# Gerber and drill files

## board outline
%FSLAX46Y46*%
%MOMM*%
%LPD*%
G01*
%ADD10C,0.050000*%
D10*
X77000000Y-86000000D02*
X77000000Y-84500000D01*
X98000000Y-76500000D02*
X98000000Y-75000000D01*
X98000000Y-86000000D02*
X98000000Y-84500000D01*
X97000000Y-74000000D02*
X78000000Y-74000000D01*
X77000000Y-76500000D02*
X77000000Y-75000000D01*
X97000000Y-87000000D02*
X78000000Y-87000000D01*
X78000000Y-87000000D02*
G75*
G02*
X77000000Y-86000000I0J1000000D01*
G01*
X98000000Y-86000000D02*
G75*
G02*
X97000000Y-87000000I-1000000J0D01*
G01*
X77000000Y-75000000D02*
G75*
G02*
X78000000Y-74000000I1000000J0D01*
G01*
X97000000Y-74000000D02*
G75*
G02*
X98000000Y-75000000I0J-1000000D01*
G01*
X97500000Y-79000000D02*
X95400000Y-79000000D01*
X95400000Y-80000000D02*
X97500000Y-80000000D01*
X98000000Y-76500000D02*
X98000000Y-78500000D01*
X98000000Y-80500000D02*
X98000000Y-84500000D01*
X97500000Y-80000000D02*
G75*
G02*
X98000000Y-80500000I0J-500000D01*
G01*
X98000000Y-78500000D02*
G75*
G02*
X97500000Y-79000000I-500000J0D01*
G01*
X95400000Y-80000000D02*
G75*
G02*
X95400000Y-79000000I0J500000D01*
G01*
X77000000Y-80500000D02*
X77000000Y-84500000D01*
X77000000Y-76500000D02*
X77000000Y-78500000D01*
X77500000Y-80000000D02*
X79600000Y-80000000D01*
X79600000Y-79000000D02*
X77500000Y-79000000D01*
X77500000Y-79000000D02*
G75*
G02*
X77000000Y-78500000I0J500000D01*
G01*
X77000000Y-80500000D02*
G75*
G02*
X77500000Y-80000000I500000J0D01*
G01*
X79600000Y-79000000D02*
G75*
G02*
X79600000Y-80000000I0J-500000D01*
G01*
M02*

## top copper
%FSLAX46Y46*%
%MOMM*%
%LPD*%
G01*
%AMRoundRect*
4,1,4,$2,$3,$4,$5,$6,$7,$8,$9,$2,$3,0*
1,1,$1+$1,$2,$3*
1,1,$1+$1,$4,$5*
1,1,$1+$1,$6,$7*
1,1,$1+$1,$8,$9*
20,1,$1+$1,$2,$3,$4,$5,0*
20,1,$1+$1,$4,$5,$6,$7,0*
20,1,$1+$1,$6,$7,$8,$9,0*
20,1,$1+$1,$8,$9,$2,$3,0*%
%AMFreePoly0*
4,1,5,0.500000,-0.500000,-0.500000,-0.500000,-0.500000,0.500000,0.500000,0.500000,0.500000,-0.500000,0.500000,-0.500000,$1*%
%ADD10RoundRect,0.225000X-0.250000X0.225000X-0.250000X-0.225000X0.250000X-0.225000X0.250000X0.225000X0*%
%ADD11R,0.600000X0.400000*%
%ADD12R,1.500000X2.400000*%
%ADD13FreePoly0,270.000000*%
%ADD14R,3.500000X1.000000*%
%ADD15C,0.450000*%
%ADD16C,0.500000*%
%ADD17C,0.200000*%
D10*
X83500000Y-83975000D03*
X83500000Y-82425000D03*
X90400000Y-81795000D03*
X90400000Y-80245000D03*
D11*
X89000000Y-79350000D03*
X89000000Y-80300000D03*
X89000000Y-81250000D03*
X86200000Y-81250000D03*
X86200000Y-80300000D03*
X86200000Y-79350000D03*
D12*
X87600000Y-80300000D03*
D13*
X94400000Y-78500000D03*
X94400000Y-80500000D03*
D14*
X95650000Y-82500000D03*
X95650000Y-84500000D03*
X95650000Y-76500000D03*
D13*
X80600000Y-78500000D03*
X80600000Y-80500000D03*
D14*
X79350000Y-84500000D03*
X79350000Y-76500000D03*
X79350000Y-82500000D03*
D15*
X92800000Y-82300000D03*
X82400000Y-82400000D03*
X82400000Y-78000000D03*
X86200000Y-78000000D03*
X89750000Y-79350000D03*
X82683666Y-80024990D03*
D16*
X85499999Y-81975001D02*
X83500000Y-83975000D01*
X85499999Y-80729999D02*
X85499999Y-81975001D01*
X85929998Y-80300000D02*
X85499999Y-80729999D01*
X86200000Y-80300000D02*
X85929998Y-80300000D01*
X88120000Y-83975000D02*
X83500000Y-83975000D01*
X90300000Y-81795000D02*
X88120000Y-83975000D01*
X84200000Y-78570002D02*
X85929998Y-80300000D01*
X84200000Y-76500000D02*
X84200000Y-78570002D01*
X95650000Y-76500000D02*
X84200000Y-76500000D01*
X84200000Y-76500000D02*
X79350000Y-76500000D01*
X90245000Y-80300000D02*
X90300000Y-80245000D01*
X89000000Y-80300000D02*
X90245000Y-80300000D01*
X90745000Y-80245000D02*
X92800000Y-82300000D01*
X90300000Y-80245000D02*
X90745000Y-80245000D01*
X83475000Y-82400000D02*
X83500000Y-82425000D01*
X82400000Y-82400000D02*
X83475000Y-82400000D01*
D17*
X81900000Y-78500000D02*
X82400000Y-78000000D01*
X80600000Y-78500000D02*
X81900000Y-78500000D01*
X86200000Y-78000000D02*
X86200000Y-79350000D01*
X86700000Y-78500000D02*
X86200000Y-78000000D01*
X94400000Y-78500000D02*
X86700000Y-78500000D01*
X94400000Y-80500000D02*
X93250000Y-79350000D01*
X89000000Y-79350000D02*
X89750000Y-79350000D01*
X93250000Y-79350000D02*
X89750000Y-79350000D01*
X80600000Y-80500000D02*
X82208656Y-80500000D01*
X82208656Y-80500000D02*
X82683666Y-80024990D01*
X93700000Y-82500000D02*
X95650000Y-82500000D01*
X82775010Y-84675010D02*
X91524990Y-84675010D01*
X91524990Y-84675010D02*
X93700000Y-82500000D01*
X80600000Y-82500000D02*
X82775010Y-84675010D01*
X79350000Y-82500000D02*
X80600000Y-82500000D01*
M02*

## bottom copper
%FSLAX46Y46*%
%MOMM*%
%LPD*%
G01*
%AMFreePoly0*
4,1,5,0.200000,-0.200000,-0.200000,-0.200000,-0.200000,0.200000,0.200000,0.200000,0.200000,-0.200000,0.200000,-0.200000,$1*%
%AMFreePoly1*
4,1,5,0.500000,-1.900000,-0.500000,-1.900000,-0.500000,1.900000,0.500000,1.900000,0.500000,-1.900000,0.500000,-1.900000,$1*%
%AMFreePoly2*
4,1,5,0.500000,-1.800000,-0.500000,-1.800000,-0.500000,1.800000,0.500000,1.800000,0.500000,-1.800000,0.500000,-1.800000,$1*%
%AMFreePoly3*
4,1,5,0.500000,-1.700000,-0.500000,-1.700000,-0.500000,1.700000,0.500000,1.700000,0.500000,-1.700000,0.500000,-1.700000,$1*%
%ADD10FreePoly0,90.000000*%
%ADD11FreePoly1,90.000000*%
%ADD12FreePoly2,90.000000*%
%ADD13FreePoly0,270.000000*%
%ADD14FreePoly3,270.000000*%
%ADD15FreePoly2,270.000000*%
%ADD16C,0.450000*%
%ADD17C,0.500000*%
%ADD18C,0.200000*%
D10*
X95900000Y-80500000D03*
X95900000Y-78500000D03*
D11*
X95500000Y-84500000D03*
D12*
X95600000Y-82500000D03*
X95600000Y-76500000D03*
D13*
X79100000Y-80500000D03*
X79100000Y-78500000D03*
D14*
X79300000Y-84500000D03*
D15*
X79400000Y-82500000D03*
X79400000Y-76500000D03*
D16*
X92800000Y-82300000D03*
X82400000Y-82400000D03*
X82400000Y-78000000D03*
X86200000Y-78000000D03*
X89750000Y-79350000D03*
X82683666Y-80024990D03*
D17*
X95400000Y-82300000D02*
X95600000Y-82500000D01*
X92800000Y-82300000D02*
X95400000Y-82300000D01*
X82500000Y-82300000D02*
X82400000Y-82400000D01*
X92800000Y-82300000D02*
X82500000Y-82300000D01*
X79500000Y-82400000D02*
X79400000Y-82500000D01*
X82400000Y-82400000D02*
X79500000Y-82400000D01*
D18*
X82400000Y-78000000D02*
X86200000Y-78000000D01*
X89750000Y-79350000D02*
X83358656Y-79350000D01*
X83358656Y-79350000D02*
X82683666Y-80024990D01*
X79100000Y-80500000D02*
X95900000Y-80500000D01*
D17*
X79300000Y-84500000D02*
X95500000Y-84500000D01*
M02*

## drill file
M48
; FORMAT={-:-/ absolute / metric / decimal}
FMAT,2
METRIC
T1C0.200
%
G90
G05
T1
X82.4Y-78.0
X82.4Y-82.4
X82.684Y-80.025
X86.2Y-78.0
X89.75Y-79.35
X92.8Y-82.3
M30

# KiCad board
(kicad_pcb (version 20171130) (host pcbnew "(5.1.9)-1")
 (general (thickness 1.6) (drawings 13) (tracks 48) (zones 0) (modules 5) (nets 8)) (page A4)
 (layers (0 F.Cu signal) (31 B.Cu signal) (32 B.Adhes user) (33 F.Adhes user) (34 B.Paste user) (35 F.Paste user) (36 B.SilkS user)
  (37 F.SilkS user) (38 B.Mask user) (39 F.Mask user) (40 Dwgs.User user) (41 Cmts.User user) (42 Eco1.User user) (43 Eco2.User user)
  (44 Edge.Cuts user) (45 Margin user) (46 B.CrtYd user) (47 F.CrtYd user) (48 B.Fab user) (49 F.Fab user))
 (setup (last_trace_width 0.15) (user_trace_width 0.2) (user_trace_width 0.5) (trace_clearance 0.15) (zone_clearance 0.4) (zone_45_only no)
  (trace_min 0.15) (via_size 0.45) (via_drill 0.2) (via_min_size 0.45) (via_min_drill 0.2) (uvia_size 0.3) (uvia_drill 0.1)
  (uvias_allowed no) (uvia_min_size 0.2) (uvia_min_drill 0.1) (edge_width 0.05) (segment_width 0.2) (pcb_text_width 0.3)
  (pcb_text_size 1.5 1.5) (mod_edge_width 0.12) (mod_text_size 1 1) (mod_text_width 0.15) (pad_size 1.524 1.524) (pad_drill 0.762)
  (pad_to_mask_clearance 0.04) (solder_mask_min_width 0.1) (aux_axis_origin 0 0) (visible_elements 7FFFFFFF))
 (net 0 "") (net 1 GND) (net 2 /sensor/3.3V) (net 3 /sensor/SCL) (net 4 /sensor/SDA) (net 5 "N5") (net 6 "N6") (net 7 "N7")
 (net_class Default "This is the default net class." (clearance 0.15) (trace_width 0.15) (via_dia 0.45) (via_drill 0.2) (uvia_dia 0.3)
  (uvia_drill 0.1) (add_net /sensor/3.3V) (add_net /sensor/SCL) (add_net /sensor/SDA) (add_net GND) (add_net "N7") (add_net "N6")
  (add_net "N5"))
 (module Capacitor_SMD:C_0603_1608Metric (layer F.Cu) (at 83.5 83.2 270)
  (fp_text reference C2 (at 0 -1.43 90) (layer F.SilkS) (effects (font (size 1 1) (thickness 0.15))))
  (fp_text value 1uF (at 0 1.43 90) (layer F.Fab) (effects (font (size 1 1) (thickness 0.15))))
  (pad 2 smd roundrect (at 0.775 0 270) (size 0.9 0.95) (layers F.Cu F.Paste F.Mask) (roundrect_rratio 0.25) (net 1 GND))
  (pad 1 smd roundrect (at -0.775 0 270) (size 0.9 0.95) (layers F.Cu F.Paste F.Mask) (roundrect_rratio 0.25) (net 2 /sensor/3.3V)))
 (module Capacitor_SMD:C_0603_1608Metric (layer F.Cu) (at 90.4 81.02 270)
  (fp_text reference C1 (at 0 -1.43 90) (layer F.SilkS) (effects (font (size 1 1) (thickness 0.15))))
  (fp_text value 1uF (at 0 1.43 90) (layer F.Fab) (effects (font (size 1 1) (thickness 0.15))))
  (pad 2 smd roundrect (at 0.775 0 270) (size 0.9 0.95) (layers F.Cu F.Paste F.Mask) (roundrect_rratio 0.25) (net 1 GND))
  (pad 1 smd roundrect (at -0.775 0 270) (size 0.9 0.95) (layers F.Cu F.Paste F.Mask) (roundrect_rratio 0.25) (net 2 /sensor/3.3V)))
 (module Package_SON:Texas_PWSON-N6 (layer F.Cu) (at 87.6 80.3)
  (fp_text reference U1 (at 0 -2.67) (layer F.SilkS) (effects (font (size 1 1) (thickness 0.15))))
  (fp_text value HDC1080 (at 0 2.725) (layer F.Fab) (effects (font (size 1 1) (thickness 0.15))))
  (pad 6 smd rect (at 1.4 -0.95) (size 0.6 0.4) (layers F.Cu F.Paste F.Mask) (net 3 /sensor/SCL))
  (pad 5 smd rect (at 1.4 0) (size 0.6 0.4) (layers F.Cu F.Paste F.Mask) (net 2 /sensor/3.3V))
  (pad 4 smd rect (at 1.4 0.95) (size 0.6 0.4) (layers F.Cu F.Paste F.Mask))
  (pad 3 smd rect (at -1.4 0.95) (size 0.6 0.4) (layers F.Cu F.Paste F.Mask))
  (pad 2 smd rect (at -1.4 0) (size 0.6 0.4) (layers F.Cu F.Paste F.Mask) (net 1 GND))
  (pad 1 smd rect (at -1.4 -0.95) (size 0.6 0.4) (layers F.Cu F.Paste F.Mask) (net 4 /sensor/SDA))
  (pad 7 smd rect (at 0 0) (size 1.5 2.4) (layers F.Cu F.Paste F.Mask)))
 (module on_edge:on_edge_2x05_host (layer F.Cu) (at 98 80.5 270)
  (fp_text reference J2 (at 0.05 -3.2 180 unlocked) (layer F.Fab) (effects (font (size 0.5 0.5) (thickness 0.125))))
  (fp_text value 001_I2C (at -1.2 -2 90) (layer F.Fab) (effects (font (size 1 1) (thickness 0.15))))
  (fp_line (start -1.5 0.5) (end -1.5 2.6) (layer Edge.Cuts) (width 0.05))
  (fp_line (start -0.5 2.6) (end -0.5 0.5) (layer Edge.Cuts) (width 0.05))
  (fp_line (start -4 0) (end -2 0) (layer Edge.Cuts) (width 0.05))
  (fp_line (start 0 0) (end 4 0) (layer Edge.Cuts) (width 0.05))
  (fp_arc (start 0 0.5) (end 0 0) (angle -90) (layer Edge.Cuts) (width 0.05))
  (fp_arc (start -2 0.5) (end -1.5 0.5) (angle -90) (layer Edge.Cuts) (width 0.05))
  (fp_arc (start -1 2.6) (end -1.5 2.6) (angle -180) (layer Edge.Cuts) (width 0.05))
  (pad 2 smd custom (at -2 3.6 270) (size 1 1) (layers F.Cu F.Mask) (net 4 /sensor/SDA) (zone_connect 0)
   (options (clearance outline) (anchor rect)) (primitives))
  (pad 3 smd custom (at 0 3.6 270) (size 1 1) (layers F.Cu F.Mask) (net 3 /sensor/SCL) (zone_connect 0)
   (options (clearance outline) (anchor rect)) (primitives))
  (pad 8 smd custom (at 0 2.1 90) (size 0.4 0.4) (layers B.Cu B.Mask) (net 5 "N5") (zone_connect 0)
   (options (clearance outline) (anchor rect)) (primitives))
  (pad 7 smd custom (at -2 2.1 90) (size 0.4 0.4) (layers B.Cu B.Mask) (zone_connect 0) (options (clearance outline) (anchor rect))
   (primitives))
  (pad 4 smd rect (at 2 2.35 270) (size 1 3.5) (layers F.Cu F.Mask) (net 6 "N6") (zone_connect 0))
  (pad 10 smd custom (at 4 2.5 90) (size 1 3.8) (layers B.Cu B.Mask) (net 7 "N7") (zone_connect 0)
   (options (clearance outline) (anchor rect)) (primitives))
  (pad 9 smd custom (at 2 2.4 90) (size 1 3.6) (layers B.Cu B.Mask) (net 2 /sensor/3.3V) (zone_connect 0)
   (options (clearance outline) (anchor rect)) (primitives))
  (pad 6 smd custom (at -4 2.4 90) (size 1 3.6) (layers B.Cu B.Mask) (zone_connect 0) (options (clearance outline) (anchor rect))
   (primitives))
  (pad 5 smd rect (at 4 2.35 270) (size 1 3.5) (layers F.Cu F.Mask) (zone_connect 0))
  (pad 1 smd rect (at -4 2.35 270) (size 1 3.5) (layers F.Cu F.Mask) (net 1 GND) (zone_connect 0)))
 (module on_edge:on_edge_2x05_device (layer F.Cu) (at 77 80.5 270)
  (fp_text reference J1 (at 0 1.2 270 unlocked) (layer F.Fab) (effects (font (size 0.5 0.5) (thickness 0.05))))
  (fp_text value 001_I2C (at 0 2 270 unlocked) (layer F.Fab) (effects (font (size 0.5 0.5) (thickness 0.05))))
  (fp_line (start 0 0) (end 4 0) (layer Edge.Cuts) (width 0.05))
  (fp_line (start -4 0) (end -2 0) (layer Edge.Cuts) (width 0.05))
  (fp_line (start -0.5 -0.5) (end -0.5 -2.6) (layer Edge.Cuts) (width 0.05))
  (fp_line (start -1.5 -2.6) (end -1.5 -0.5) (layer Edge.Cuts) (width 0.05))
  (fp_arc (start -2 -0.5) (end -2 0) (angle -90) (layer Edge.Cuts) (width 0.05))
  (fp_arc (start 0 -0.5) (end -0.5 -0.5) (angle -90) (layer Edge.Cuts) (width 0.05))
  (fp_arc (start -1 -2.6) (end -0.5 -2.6) (angle -180) (layer Edge.Cuts) (width 0.05))
  (pad 2 smd custom (at -2 -3.6 270) (size 1 1) (layers F.Cu F.Mask) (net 4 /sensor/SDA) (zone_connect 0)
   (options (clearance outline) (anchor rect)) (primitives))
  (pad 3 smd custom (at 0 -3.6 270) (size 1 1) (layers F.Cu F.Mask) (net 3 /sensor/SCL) (zone_connect 0)
   (options (clearance outline) (anchor rect)) (primitives))
  (pad 8 smd custom (at 0 -2.1 270) (size 0.4 0.4) (layers B.Cu B.Mask) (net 5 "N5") (zone_connect 0)
   (options (clearance outline) (anchor rect)) (primitives))
  (pad 7 smd custom (at -2 -2.1 270) (size 0.4 0.4) (layers B.Cu B.Mask) (zone_connect 0) (options (clearance outline) (anchor rect))
   (primitives))
  (pad 10 smd custom (at 4 -2.3 270) (size 1 3.4) (layers B.Cu B.Mask) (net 7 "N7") (zone_connect 0)
   (options (clearance outline) (anchor rect)) (primitives))
  (pad 9 smd custom (at 2 -2.4 270) (size 1 3.6) (layers B.Cu B.Mask) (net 2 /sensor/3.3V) (zone_connect 0)
   (options (clearance outline) (anchor rect)) (primitives))
  (pad 6 smd custom (at -4 -2.4 270) (size 1 3.6) (layers B.Cu B.Mask) (zone_connect 0) (options (clearance outline) (anchor rect))
   (primitives))
  (pad 5 smd rect (at 4 -2.35 90) (size 1 3.5) (layers F.Cu F.Mask) (zone_connect 0))
  (pad 1 smd rect (at -4 -2.35 90) (size 1 3.5) (layers F.Cu F.Mask) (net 1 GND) (zone_connect 0))
  (pad 4 smd rect (at 2 -2.35 90) (size 1 3.5) (layers F.Cu F.Mask) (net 6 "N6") (zone_connect 0)))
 (gr_line (start 77 86) (end 77 84.5) (layer Edge.Cuts) (width 0.05))
 (gr_line (start 98 76.5) (end 98 75) (layer Edge.Cuts) (width 0.05))
 (gr_line (start 98 86) (end 98 84.5) (layer Edge.Cuts) (width 0.05))
 (gr_line (start 97 74) (end 78 74) (layer Edge.Cuts) (width 0.05))
 (gr_line (start 77 76.5) (end 77 75) (layer Edge.Cuts) (width 0.05))
 (gr_line (start 97 87) (end 78 87) (layer Edge.Cuts) (width 0.05))
 (gr_arc (start 78 86) (end 77 86) (angle -90) (layer Edge.Cuts) (width 0.05))
 (gr_arc (start 97 86) (end 97 87) (angle -90) (layer Edge.Cuts) (width 0.05))
 (gr_arc (start 78 75) (end 78 74) (angle -90) (layer Edge.Cuts) (width 0.05))
 (gr_arc (start 97 75) (end 98 75) (angle -90) (layer Edge.Cuts) (width 0.05))
 (segment (start 85.499999 81.975001) (end 83.5 83.975) (width 0.5) (layer F.Cu) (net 1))
 (segment (start 85.499999 80.729999) (end 85.499999 81.975001) (width 0.5) (layer F.Cu) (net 1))
 (segment (start 85.929998 80.3) (end 85.499999 80.729999) (width 0.5) (layer F.Cu) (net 1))
 (segment (start 86.2 80.3) (end 85.929998 80.3) (width 0.5) (layer F.Cu) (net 1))
 (segment (start 88.12 83.975) (end 83.5 83.975) (width 0.5) (layer F.Cu) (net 1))
 (segment (start 90.3 81.795) (end 88.12 83.975) (width 0.5) (layer F.Cu) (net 1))
 (segment (start 84.2 78.570002) (end 85.929998 80.3) (width 0.5) (layer F.Cu) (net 1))
 (segment (start 84.2 76.5) (end 84.2 78.570002) (width 0.5) (layer F.Cu) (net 1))
 (segment (start 95.65 76.5) (end 84.2 76.5) (width 0.5) (layer F.Cu) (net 1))
 (segment (start 84.2 76.5) (end 79.35 76.5) (width 0.5) (layer F.Cu) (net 1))
 (segment (start 90.245 80.3) (end 90.3 80.245) (width 0.5) (layer F.Cu) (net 2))
 (segment (start 89 80.3) (end 90.245 80.3) (width 0.5) (layer F.Cu) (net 2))
 (via (at 92.8 82.3) (size 0.45) (drill 0.2) (layers F.Cu B.Cu) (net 2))
 (segment (start 90.745 80.245) (end 92.8 82.3) (width 0.5) (layer F.Cu) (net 2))
 (segment (start 90.3 80.245) (end 90.745 80.245) (width 0.5) (layer F.Cu) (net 2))
 (segment (start 95.4 82.3) (end 95.6 82.5) (width 0.5) (layer B.Cu) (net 2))
 (segment (start 92.8 82.3) (end 95.4 82.3) (width 0.5) (layer B.Cu) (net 2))
 (via (at 82.4 82.4) (size 0.45) (drill 0.2) (layers F.Cu B.Cu) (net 2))
 (segment (start 82.5 82.3) (end 82.4 82.4) (width 0.5) (layer B.Cu) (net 2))
 (segment (start 92.8 82.3) (end 82.5 82.3) (width 0.5) (layer B.Cu) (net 2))
 (segment (start 83.475 82.4) (end 83.5 82.425) (width 0.5) (layer F.Cu) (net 2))
 (segment (start 82.4 82.4) (end 83.475 82.4) (width 0.5) (layer F.Cu) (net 2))
 (segment (start 79.5 82.4) (end 79.4 82.5) (width 0.5) (layer B.Cu) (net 2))
 (segment (start 82.4 82.4) (end 79.5 82.4) (width 0.5) (layer B.Cu) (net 2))
 (via (at 82.4 78) (size 0.45) (drill 0.2) (layers F.Cu B.Cu) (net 4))
 (segment (start 81.9 78.5) (end 82.4 78) (width 0.2) (layer F.Cu) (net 4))
 (segment (start 80.6 78.5) (end 81.9 78.5) (width 0.2) (layer F.Cu) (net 4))
 (via (at 86.2 78) (size 0.45) (drill 0.2) (layers F.Cu B.Cu) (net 4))
 (segment (start 82.4 78) (end 86.2 78) (width 0.2) (layer B.Cu) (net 4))
 (segment (start 86.2 78) (end 86.2 79.35) (width 0.2) (layer F.Cu) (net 4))
 (segment (start 86.7 78.5) (end 86.2 78) (width 0.2) (layer F.Cu) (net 4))
 (segment (start 94.4 78.5) (end 86.7 78.5) (width 0.2) (layer F.Cu) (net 4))
 (segment (start 94.4 80.5) (end 93.25 79.35) (width 0.2) (layer F.Cu) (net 3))
 (via (at 89.75 79.35) (size 0.45) (drill 0.2) (layers F.Cu B.Cu) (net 3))
 (segment (start 89 79.35) (end 89.75 79.35) (width 0.2) (layer F.Cu) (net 3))
 (segment (start 93.25 79.35) (end 89.75 79.35) (width 0.2) (layer F.Cu) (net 3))
 (via (at 82.683666 80.02499) (size 0.45) (drill 0.2) (layers F.Cu B.Cu) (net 3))
 (segment (start 89.75 79.35) (end 83.358656 79.35) (width 0.2) (layer B.Cu) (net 3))
 (segment (start 83.358656 79.35) (end 82.683666 80.02499) (width 0.2) (layer B.Cu) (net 3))
 (segment (start 80.6 80.5) (end 82.208656 80.5) (width 0.2) (layer F.Cu) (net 3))
 (segment (start 82.208656 80.5) (end 82.683666 80.02499) (width 0.2) (layer F.Cu) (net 3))
 (segment (start 79.1 80.5) (end 95.9 80.5) (width 0.2) (layer B.Cu) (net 5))
 (segment (start 79.3 84.5) (end 95.5 84.5) (width 0.5) (layer B.Cu) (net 7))
 (segment (start 93.7 82.5) (end 95.65 82.5) (width 0.2) (layer F.Cu) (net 6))
 (segment (start 82.77501 84.67501) (end 91.52499 84.67501) (width 0.2) (layer F.Cu) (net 6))
 (segment (start 91.52499 84.67501) (end 93.7 82.5) (width 0.2) (layer F.Cu) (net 6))
 (segment (start 80.6 82.5) (end 82.77501 84.67501) (width 0.2) (layer F.Cu) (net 6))
 (segment (start 79.35 82.5) (end 80.6 82.5) (width 0.2) (layer F.Cu) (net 6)))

